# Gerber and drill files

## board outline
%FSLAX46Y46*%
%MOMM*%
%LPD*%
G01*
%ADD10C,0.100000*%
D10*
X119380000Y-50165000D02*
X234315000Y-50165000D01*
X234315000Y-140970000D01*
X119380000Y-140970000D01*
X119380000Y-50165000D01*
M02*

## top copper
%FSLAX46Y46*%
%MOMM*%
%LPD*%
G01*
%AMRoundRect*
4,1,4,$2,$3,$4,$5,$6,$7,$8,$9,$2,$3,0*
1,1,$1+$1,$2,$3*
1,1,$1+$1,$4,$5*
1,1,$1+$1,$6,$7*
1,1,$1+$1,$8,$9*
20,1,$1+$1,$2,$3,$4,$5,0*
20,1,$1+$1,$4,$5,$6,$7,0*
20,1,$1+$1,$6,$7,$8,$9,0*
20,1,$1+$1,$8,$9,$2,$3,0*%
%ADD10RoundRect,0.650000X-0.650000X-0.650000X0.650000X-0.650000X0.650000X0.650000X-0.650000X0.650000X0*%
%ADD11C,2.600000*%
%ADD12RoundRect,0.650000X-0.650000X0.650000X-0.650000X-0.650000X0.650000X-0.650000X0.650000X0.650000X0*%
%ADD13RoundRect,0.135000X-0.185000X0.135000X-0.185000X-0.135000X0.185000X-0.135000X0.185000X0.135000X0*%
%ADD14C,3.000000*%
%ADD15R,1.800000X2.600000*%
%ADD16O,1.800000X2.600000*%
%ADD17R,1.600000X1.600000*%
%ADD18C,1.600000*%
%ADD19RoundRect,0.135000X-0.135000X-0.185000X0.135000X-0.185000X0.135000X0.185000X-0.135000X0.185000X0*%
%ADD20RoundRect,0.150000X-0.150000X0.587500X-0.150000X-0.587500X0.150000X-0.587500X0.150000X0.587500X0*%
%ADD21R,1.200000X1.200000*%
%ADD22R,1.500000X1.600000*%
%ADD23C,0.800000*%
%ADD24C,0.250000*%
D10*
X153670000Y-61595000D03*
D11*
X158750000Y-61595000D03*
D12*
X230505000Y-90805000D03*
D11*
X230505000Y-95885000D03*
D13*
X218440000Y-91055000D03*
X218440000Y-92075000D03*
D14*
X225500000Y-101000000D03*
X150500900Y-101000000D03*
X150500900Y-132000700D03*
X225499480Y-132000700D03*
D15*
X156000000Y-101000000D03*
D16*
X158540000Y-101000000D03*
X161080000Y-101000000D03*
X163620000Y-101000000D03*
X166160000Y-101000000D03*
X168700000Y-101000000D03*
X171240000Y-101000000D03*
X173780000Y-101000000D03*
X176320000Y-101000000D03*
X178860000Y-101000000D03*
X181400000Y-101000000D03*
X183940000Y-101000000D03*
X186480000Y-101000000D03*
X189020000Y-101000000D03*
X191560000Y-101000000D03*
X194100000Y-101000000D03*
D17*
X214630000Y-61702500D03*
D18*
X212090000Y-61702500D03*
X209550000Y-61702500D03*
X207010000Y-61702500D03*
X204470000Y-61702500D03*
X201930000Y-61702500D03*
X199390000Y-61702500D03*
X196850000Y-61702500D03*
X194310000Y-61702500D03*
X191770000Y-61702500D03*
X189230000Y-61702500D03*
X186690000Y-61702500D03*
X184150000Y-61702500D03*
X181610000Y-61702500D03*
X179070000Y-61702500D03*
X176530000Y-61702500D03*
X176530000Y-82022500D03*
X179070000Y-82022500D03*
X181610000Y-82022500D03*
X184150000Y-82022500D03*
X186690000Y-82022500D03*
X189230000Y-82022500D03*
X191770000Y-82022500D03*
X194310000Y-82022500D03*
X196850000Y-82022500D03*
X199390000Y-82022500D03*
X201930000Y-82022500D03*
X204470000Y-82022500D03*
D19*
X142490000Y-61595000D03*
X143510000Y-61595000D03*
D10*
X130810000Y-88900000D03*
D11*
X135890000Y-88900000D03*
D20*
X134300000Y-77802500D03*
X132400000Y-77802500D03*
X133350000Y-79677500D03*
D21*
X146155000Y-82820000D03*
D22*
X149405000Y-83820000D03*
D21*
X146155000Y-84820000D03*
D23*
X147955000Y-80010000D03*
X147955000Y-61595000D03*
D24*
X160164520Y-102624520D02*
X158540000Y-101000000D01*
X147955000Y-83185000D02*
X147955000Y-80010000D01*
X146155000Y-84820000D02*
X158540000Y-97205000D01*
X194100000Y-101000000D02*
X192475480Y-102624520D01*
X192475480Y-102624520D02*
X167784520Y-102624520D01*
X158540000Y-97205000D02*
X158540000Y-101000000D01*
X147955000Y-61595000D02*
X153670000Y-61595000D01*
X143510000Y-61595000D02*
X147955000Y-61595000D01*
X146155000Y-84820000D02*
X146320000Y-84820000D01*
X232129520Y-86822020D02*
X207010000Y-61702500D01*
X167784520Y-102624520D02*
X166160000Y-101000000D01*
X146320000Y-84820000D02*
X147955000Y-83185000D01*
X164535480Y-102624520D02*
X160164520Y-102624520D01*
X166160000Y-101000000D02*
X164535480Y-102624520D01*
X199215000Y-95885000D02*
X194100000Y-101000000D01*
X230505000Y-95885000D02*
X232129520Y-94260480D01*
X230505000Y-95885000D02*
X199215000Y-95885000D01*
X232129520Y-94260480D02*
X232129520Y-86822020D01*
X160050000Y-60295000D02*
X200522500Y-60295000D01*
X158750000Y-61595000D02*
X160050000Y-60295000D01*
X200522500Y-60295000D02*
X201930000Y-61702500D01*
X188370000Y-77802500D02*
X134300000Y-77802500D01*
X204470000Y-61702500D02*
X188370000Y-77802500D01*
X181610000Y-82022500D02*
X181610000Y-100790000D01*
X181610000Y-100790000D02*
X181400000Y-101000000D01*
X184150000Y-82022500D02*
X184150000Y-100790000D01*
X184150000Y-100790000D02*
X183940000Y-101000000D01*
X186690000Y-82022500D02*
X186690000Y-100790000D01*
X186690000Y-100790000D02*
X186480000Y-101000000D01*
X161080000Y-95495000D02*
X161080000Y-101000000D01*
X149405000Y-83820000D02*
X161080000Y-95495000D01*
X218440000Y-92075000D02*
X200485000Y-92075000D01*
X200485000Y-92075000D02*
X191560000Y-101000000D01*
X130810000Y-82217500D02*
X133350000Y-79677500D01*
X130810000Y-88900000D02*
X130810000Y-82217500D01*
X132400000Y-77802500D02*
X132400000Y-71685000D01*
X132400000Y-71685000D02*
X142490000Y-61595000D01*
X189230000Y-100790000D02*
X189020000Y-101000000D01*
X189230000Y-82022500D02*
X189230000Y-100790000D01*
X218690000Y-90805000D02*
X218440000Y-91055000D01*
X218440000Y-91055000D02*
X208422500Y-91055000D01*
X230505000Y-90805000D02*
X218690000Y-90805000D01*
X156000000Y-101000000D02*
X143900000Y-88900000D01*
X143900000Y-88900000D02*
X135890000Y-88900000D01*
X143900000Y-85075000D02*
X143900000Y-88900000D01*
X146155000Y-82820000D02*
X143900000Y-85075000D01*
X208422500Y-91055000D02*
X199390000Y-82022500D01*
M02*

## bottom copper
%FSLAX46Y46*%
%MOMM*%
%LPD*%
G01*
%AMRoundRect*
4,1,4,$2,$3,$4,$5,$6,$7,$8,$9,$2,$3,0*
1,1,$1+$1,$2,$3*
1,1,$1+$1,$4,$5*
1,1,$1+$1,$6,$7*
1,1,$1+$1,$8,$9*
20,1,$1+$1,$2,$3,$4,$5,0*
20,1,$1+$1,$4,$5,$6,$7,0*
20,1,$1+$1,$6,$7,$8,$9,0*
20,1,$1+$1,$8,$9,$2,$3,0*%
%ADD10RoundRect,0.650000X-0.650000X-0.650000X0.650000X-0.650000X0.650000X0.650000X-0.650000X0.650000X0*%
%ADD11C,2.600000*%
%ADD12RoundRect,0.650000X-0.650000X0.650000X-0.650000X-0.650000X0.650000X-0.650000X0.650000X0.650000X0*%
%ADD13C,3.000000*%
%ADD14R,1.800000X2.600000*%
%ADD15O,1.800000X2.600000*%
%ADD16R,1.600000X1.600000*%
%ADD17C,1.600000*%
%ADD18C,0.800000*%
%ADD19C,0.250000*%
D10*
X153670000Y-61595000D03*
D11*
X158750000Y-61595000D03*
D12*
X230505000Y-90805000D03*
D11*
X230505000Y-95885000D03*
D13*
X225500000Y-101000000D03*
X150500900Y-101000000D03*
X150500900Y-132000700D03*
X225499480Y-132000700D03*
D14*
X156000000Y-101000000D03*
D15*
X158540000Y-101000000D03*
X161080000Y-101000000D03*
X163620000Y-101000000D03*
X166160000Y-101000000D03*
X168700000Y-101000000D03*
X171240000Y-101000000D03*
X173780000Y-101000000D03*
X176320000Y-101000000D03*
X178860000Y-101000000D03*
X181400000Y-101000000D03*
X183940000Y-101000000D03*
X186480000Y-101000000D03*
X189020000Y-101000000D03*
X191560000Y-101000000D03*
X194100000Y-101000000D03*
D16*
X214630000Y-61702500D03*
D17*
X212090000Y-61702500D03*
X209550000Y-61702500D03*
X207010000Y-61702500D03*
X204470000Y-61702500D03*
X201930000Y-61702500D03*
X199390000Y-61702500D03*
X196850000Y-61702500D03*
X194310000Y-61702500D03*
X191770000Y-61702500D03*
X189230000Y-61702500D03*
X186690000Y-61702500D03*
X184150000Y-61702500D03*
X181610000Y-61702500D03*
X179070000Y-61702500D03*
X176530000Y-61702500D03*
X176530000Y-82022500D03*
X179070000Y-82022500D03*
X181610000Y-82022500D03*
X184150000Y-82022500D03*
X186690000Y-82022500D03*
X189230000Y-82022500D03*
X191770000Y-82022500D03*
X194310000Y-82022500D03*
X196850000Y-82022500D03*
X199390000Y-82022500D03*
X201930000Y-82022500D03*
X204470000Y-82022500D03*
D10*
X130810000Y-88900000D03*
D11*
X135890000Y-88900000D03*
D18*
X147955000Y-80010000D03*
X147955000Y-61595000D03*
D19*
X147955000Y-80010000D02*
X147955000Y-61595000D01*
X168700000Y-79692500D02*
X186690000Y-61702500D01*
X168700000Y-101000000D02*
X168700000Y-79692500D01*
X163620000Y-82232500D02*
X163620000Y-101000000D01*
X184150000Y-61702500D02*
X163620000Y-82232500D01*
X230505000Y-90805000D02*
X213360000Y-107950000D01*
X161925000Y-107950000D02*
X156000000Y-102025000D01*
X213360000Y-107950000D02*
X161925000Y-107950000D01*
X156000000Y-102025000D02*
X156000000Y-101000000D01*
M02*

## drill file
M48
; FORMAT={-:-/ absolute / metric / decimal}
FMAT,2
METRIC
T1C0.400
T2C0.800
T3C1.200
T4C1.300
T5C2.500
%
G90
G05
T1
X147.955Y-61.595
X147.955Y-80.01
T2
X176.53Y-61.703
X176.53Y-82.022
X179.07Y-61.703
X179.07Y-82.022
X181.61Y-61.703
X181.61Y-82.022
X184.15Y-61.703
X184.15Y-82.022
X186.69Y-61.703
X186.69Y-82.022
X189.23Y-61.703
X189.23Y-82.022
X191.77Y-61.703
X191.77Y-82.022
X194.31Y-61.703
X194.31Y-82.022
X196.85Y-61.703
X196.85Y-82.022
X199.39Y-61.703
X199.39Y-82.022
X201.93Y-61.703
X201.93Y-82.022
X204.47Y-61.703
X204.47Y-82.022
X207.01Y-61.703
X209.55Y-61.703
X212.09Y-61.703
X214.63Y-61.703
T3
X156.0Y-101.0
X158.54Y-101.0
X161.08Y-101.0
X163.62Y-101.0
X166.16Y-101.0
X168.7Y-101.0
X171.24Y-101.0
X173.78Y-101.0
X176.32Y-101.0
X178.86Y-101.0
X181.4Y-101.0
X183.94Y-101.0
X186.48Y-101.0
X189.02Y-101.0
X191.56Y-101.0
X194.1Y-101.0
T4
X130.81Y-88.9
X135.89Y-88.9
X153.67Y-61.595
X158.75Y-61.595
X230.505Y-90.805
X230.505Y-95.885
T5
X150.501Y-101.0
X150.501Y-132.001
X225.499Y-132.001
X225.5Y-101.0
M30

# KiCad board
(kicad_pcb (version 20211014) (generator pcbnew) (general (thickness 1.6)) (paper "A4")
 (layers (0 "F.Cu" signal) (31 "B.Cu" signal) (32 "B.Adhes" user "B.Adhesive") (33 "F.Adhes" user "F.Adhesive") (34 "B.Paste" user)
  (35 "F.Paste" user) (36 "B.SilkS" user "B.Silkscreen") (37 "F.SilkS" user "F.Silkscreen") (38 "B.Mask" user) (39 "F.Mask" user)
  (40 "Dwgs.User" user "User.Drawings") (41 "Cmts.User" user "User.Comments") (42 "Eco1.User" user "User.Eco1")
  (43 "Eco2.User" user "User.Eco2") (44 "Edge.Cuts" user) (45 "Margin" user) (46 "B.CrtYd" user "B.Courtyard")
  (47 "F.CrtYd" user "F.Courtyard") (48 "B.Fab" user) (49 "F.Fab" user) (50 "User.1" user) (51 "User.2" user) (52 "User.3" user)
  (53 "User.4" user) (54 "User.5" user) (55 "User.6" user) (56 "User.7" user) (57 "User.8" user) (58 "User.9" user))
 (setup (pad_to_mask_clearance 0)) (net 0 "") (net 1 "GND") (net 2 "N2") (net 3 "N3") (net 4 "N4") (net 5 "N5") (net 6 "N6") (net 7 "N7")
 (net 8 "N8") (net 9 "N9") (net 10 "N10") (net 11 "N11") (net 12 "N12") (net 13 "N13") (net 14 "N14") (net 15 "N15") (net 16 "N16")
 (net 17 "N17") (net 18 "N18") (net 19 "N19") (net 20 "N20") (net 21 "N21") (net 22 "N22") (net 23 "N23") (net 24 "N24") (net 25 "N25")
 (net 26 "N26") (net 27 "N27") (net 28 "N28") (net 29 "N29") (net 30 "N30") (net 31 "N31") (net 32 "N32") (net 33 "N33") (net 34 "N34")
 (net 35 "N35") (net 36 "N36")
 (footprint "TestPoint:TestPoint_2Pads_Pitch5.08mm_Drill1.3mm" (layer "F.Cu") (at 153.67 61.595)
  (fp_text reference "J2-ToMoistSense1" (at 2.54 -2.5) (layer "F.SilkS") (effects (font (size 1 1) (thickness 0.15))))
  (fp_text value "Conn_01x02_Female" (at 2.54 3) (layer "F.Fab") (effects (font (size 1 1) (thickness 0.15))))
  (pad "1" thru_hole roundrect (at 0 0) (size 2.6 2.6) (drill 1.3) (layers *.Cu *.Mask) (roundrect_rratio 0.25) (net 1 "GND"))
  (pad "2" thru_hole circle (at 5.08 0) (size 2.6 2.6) (drill 1.3) (layers *.Cu *.Mask) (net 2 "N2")))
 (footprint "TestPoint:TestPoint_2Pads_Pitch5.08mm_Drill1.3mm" (layer "F.Cu") (at 230.505 90.805 -90)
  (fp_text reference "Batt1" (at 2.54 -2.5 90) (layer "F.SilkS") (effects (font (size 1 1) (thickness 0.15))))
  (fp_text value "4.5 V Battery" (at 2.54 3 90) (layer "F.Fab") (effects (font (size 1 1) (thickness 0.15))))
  (pad "1" thru_hole roundrect (at 0 0 270) (size 2.6 2.6) (drill 1.3) (layers *.Cu *.Mask) (roundrect_rratio 0.25) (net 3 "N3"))
  (pad "2" thru_hole circle (at 5.08 0 270) (size 2.6 2.6) (drill 1.3) (layers *.Cu *.Mask) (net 1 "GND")))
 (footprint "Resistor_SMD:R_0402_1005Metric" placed (layer "F.Cu") (at 218.44 91.565 -90)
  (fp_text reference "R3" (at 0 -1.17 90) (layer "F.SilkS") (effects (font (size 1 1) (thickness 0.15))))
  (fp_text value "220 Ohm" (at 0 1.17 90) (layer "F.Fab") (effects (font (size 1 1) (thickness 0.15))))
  (pad "1" smd roundrect (at -0.51 0 270) (size 0.54 0.64) (layers "F.Cu" "F.Paste" "F.Mask") (roundrect_rratio 0.25) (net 3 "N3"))
  (pad "2" smd roundrect (at 0.51 0 270) (size 0.54 0.64) (layers "F.Cu" "F.Paste" "F.Mask") (roundrect_rratio 0.25) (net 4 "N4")))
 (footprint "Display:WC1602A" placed (layer "F.Cu") (at 156 101)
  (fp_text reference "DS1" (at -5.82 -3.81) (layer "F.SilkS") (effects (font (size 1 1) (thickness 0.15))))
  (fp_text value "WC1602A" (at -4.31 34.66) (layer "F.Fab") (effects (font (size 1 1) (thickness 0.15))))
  (pad "" thru_hole circle (at 69.5 0) (size 3 3) (drill 2.5) (layers *.Cu *.Mask))
  (pad "" thru_hole circle (at -5.4991 0) (size 3 3) (drill 2.5) (layers *.Cu *.Mask))
  (pad "" thru_hole circle (at -5.4991 31.0007) (size 3 3) (drill 2.5) (layers *.Cu *.Mask))
  (pad "" thru_hole circle (at 69.49948 31.0007) (size 3 3) (drill 2.5) (layers *.Cu *.Mask))
  (pad "1" thru_hole rect (at 0 0) (size 1.8 2.6) (drill 1.2) (layers *.Cu *.Mask) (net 3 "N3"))
  (pad "2" thru_hole oval (at 2.54 0) (size 1.8 2.6) (drill 1.2) (layers *.Cu *.Mask) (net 1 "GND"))
  (pad "3" thru_hole oval (at 5.08 0) (size 1.8 2.6) (drill 1.2) (layers *.Cu *.Mask) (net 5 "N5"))
  (pad "4" thru_hole oval (at 7.62 0) (size 1.8 2.6) (drill 1.2) (layers *.Cu *.Mask) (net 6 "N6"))
  (pad "5" thru_hole oval (at 10.16 0) (size 1.8 2.6) (drill 1.2) (layers *.Cu *.Mask) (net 1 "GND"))
  (pad "6" thru_hole oval (at 12.7 0) (size 1.8 2.6) (drill 1.2) (layers *.Cu *.Mask) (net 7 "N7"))
  (pad "7" thru_hole oval (at 15.24 0) (size 1.8 2.6) (drill 1.2) (layers *.Cu *.Mask) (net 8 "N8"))
  (pad "8" thru_hole oval (at 17.78 0) (size 1.8 2.6) (drill 1.2) (layers *.Cu *.Mask) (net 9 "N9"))
  (pad "9" thru_hole oval (at 20.32 0) (size 1.8 2.6) (drill 1.2) (layers *.Cu *.Mask) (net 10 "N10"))
  (pad "10" thru_hole oval (at 22.86 0) (size 1.8 2.6) (drill 1.2) (layers *.Cu *.Mask) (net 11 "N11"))
  (pad "11" thru_hole oval (at 25.4 0) (size 1.8 2.6) (drill 1.2) (layers *.Cu *.Mask) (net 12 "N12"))
  (pad "12" thru_hole oval (at 27.94 0) (size 1.8 2.6) (drill 1.2) (layers *.Cu *.Mask) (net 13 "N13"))
  (pad "13" thru_hole oval (at 30.48 0) (size 1.8 2.6) (drill 1.2) (layers *.Cu *.Mask) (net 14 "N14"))
  (pad "14" thru_hole oval (at 33.02 0) (size 1.8 2.6) (drill 1.2) (layers *.Cu *.Mask) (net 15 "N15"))
  (pad "15" thru_hole oval (at 35.56 0) (size 1.8 2.6) (drill 1.2) (layers *.Cu *.Mask) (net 4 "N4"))
  (pad "16" thru_hole oval (at 38.1 0) (size 1.8 2.6) (drill 1.2) (layers *.Cu *.Mask) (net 1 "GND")))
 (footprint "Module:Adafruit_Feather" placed (layer "F.Cu") (at 214.63 61.7025 -90)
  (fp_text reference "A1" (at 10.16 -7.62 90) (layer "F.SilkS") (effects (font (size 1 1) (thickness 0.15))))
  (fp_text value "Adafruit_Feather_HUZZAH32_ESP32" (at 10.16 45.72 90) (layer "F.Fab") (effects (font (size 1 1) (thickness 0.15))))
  (pad "1" thru_hole rect (at 0 0 90) (size 1.6 1.6) (drill 0.8) (layers *.Cu *.Mask) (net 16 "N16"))
  (pad "2" thru_hole circle (at 0 2.54 90) (size 1.6 1.6) (drill 0.8) (layers *.Cu *.Mask) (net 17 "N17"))
  (pad "3" thru_hole circle (at 0 5.08 90) (size 1.6 1.6) (drill 0.8) (layers *.Cu *.Mask) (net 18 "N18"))
  (pad "4" thru_hole circle (at 0 7.62 90) (size 1.6 1.6) (drill 0.8) (layers *.Cu *.Mask) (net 1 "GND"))
  (pad "5" thru_hole circle (at 0 10.16 90) (size 1.6 1.6) (drill 0.8) (layers *.Cu *.Mask) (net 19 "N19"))
  (pad "6" thru_hole circle (at 0 12.7 90) (size 1.6 1.6) (drill 0.8) (layers *.Cu *.Mask) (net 2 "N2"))
  (pad "7" thru_hole circle (at 0 15.24 90) (size 1.6 1.6) (drill 0.8) (layers *.Cu *.Mask) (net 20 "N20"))
  (pad "8" thru_hole circle (at 0 17.78 90) (size 1.6 1.6) (drill 0.8) (layers *.Cu *.Mask) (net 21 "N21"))
  (pad "9" thru_hole circle (at 0 20.32 90) (size 1.6 1.6) (drill 0.8) (layers *.Cu *.Mask) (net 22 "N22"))
  (pad "10" thru_hole circle (at 0 22.86 90) (size 1.6 1.6) (drill 0.8) (layers *.Cu *.Mask) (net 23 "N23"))
  (pad "11" thru_hole circle (at 0 25.4 90) (size 1.6 1.6) (drill 0.8) (layers *.Cu *.Mask) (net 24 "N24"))
  (pad "12" thru_hole circle (at 0 27.94 90) (size 1.6 1.6) (drill 0.8) (layers *.Cu *.Mask) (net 7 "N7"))
  (pad "13" thru_hole circle (at 0 30.48 90) (size 1.6 1.6) (drill 0.8) (layers *.Cu *.Mask) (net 6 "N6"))
  (pad "14" thru_hole circle (at 0 33.02 90) (size 1.6 1.6) (drill 0.8) (layers *.Cu *.Mask) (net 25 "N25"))
  (pad "15" thru_hole circle (at 0 35.56 90) (size 1.6 1.6) (drill 0.8) (layers *.Cu *.Mask) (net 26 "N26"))
  (pad "16" thru_hole circle (at 0 38.1 90) (size 1.6 1.6) (drill 0.8) (layers *.Cu *.Mask) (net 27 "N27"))
  (pad "17" thru_hole circle (at 20.32 38.1 90) (size 1.6 1.6) (drill 0.8) (layers *.Cu *.Mask) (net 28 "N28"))
  (pad "18" thru_hole circle (at 20.32 35.56 90) (size 1.6 1.6) (drill 0.8) (layers *.Cu *.Mask) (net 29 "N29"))
  (pad "19" thru_hole circle (at 20.32 33.02 90) (size 1.6 1.6) (drill 0.8) (layers *.Cu *.Mask) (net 12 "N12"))
  (pad "20" thru_hole circle (at 20.32 30.48 90) (size 1.6 1.6) (drill 0.8) (layers *.Cu *.Mask) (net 13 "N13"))
  (pad "21" thru_hole circle (at 20.32 27.94 90) (size 1.6 1.6) (drill 0.8) (layers *.Cu *.Mask) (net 14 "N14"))
  (pad "22" thru_hole circle (at 20.32 25.4 90) (size 1.6 1.6) (drill 0.8) (layers *.Cu *.Mask) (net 15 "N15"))
  (pad "23" thru_hole circle (at 20.32 22.86 90) (size 1.6 1.6) (drill 0.8) (layers *.Cu *.Mask) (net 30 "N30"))
  (pad "24" thru_hole circle (at 20.32 20.32 90) (size 1.6 1.6) (drill 0.8) (layers *.Cu *.Mask) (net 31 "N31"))
  (pad "25" thru_hole circle (at 20.32 17.78 90) (size 1.6 1.6) (drill 0.8) (layers *.Cu *.Mask) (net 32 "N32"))
  (pad "26" thru_hole circle (at 20.32 15.24 90) (size 1.6 1.6) (drill 0.8) (layers *.Cu *.Mask) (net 3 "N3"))
  (pad "27" thru_hole circle (at 20.32 12.7 90) (size 1.6 1.6) (drill 0.8) (layers *.Cu *.Mask) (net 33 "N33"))
  (pad "28" thru_hole circle (at 20.32 10.16 90) (size 1.6 1.6) (drill 0.8) (layers *.Cu *.Mask) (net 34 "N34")))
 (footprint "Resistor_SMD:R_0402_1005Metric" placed (layer "F.Cu") (at 143 61.595)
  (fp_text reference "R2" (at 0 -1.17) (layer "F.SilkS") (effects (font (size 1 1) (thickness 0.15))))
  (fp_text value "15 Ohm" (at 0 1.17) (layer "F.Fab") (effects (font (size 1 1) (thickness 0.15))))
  (pad "1" smd roundrect (at -0.51 0) (size 0.54 0.64) (layers "F.Cu" "F.Paste" "F.Mask") (roundrect_rratio 0.25) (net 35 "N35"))
  (pad "2" smd roundrect (at 0.51 0) (size 0.54 0.64) (layers "F.Cu" "F.Paste" "F.Mask") (roundrect_rratio 0.25) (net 1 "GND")))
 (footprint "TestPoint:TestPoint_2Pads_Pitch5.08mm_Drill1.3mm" (layer "F.Cu") (at 130.81 88.9)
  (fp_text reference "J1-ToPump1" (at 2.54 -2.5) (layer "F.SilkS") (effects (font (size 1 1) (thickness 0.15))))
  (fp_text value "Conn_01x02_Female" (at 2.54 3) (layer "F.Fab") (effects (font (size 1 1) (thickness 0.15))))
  (pad "1" thru_hole roundrect (at 0 0) (size 2.6 2.6) (drill 1.3) (layers *.Cu *.Mask) (roundrect_rratio 0.25) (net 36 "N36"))
  (pad "2" thru_hole circle (at 5.08 0) (size 2.6 2.6) (drill 1.3) (layers *.Cu *.Mask) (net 3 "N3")))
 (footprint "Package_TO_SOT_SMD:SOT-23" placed (layer "F.Cu") (at 133.35 78.74 -90)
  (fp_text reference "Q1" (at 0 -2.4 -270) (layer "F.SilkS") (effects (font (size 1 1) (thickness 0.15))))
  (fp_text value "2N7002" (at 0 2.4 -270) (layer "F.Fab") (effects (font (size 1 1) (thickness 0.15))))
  (pad "1" smd roundrect (at -0.9375 -0.95 270) (size 1.475 0.6) (layers "F.Cu" "F.Paste" "F.Mask") (roundrect_rratio 0.25) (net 19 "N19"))
  (pad "2" smd roundrect (at -0.9375 0.95 270) (size 1.475 0.6) (layers "F.Cu" "F.Paste" "F.Mask") (roundrect_rratio 0.25) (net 35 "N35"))
  (pad "3" smd roundrect (at 0.9375 0 270) (size 1.475 0.6) (layers "F.Cu" "F.Paste" "F.Mask") (roundrect_rratio 0.25) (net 36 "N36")))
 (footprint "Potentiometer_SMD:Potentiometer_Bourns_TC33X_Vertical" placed (layer "F.Cu") (at 147.955 83.82)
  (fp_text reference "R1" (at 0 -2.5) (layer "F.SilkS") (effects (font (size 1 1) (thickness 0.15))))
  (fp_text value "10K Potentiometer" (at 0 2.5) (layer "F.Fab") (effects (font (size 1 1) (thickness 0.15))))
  (pad "1" smd rect (at -1.8 -1) (size 1.2 1.2) (layers "F.Cu" "F.Paste" "F.Mask") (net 3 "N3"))
  (pad "2" smd rect (at 1.45 0) (size 1.5 1.6) (layers "F.Cu" "F.Paste" "F.Mask") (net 5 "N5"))
  (pad "3" smd rect (at -1.8 1) (size 1.2 1.2) (layers "F.Cu" "F.Paste" "F.Mask") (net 1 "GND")))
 (gr_rect (start 119.38 140.97) (end 234.315 50.165) (layer "Edge.Cuts") (width 0.1) (fill none))
 (segment (start 160.16452 102.62452) (end 158.54 101) (width 0.25) (layer "F.Cu") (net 1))
 (segment (start 147.955 83.185) (end 147.955 80.01) (width 0.25) (layer "F.Cu") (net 1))
 (segment (start 146.155 84.82) (end 158.54 97.205) (width 0.25) (layer "F.Cu") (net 1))
 (segment (start 194.1 101) (end 192.47548 102.62452) (width 0.25) (layer "F.Cu") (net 1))
 (segment (start 192.47548 102.62452) (end 167.78452 102.62452) (width 0.25) (layer "F.Cu") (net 1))
 (segment (start 158.54 97.205) (end 158.54 101) (width 0.25) (layer "F.Cu") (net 1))
 (segment (start 147.955 61.595) (end 153.67 61.595) (width 0.25) (layer "F.Cu") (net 1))
 (segment (start 143.51 61.595) (end 147.955 61.595) (width 0.25) (layer "F.Cu") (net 1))
 (segment (start 146.155 84.82) (end 146.32 84.82) (width 0.25) (layer "F.Cu") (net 1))
 (segment (start 232.12952 86.82202) (end 207.01 61.7025) (width 0.25) (layer "F.Cu") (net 1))
 (segment (start 167.78452 102.62452) (end 166.16 101) (width 0.25) (layer "F.Cu") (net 1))
 (segment (start 146.32 84.82) (end 147.955 83.185) (width 0.25) (layer "F.Cu") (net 1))
 (segment (start 164.53548 102.62452) (end 160.16452 102.62452) (width 0.25) (layer "F.Cu") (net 1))
 (segment (start 166.16 101) (end 164.53548 102.62452) (width 0.25) (layer "F.Cu") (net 1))
 (segment (start 199.215 95.885) (end 194.1 101) (width 0.25) (layer "F.Cu") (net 1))
 (segment (start 230.505 95.885) (end 232.12952 94.26048) (width 0.25) (layer "F.Cu") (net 1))
 (segment (start 230.505 95.885) (end 199.215 95.885) (width 0.25) (layer "F.Cu") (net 1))
 (segment (start 232.12952 94.26048) (end 232.12952 86.82202) (width 0.25) (layer "F.Cu") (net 1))
 (via (at 147.955 80.01) (size 0.8) (drill 0.4) (layers "F.Cu" "B.Cu") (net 1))
 (via (at 147.955 61.595) (size 0.8) (drill 0.4) (layers "F.Cu" "B.Cu") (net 1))
 (segment (start 147.955 80.01) (end 147.955 61.595) (width 0.25) (layer "B.Cu") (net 1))
 (segment (start 160.05 60.295) (end 200.5225 60.295) (width 0.25) (layer "F.Cu") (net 2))
 (segment (start 158.75 61.595) (end 160.05 60.295) (width 0.25) (layer "F.Cu") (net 2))
 (segment (start 200.5225 60.295) (end 201.93 61.7025) (width 0.25) (layer "F.Cu") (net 2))
 (segment (start 188.37 77.8025) (end 134.3 77.8025) (width 0.25) (layer "F.Cu") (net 19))
 (segment (start 204.47 61.7025) (end 188.37 77.8025) (width 0.25) (layer "F.Cu") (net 19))
 (segment (start 181.61 82.0225) (end 181.61 100.79) (width 0.25) (layer "F.Cu") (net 12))
 (segment (start 181.61 100.79) (end 181.4 101) (width 0.25) (layer "F.Cu") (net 12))
 (segment (start 184.15 82.0225) (end 184.15 100.79) (width 0.25) (layer "F.Cu") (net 13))
 (segment (start 184.15 100.79) (end 183.94 101) (width 0.25) (layer "F.Cu") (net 13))
 (segment (start 186.69 82.0225) (end 186.69 100.79) (width 0.25) (layer "F.Cu") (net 14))
 (segment (start 186.69 100.79) (end 186.48 101) (width 0.25) (layer "F.Cu") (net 14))
 (segment (start 161.08 95.495) (end 161.08 101) (width 0.25) (layer "F.Cu") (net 5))
 (segment (start 149.405 83.82) (end 161.08 95.495) (width 0.25) (layer "F.Cu") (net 5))
 (segment (start 218.44 92.075) (end 200.485 92.075) (width 0.25) (layer "F.Cu") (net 4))
 (segment (start 200.485 92.075) (end 191.56 101) (width 0.25) (layer "F.Cu") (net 4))
 (segment (start 130.81 82.2175) (end 133.35 79.6775) (width 0.25) (layer "F.Cu") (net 36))
 (segment (start 130.81 88.9) (end 130.81 82.2175) (width 0.25) (layer "F.Cu") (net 36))
 (segment (start 132.4 77.8025) (end 132.4 71.685) (width 0.25) (layer "F.Cu") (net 35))
 (segment (start 132.4 71.685) (end 142.49 61.595) (width 0.25) (layer "F.Cu") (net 35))
 (segment (start 168.7 79.6925) (end 186.69 61.7025) (width 0.25) (layer "B.Cu") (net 7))
 (segment (start 168.7 101) (end 168.7 79.6925) (width 0.25) (layer "B.Cu") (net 7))
 (segment (start 163.62 82.2325) (end 163.62 101) (width 0.25) (layer "B.Cu") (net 6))
 (segment (start 184.15 61.7025) (end 163.62 82.2325) (width 0.25) (layer "B.Cu") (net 6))
 (segment (start 189.23 100.79) (end 189.02 101) (width 0.25) (layer "F.Cu") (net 15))
 (segment (start 189.23 82.0225) (end 189.23 100.79) (width 0.25) (layer "F.Cu") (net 15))
 (segment (start 218.69 90.805) (end 218.44 91.055) (width 0.25) (layer "F.Cu") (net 3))
 (segment (start 218.44 91.055) (end 208.4225 91.055) (width 0.25) (layer "F.Cu") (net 3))
 (segment (start 230.505 90.805) (end 218.69 90.805) (width 0.25) (layer "F.Cu") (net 3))
 (segment (start 156 101) (end 143.9 88.9) (width 0.25) (layer "F.Cu") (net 3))
 (segment (start 143.9 88.9) (end 135.89 88.9) (width 0.25) (layer "F.Cu") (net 3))
 (segment (start 143.9 85.075) (end 143.9 88.9) (width 0.25) (layer "F.Cu") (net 3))
 (segment (start 146.155 82.82) (end 143.9 85.075) (width 0.25) (layer "F.Cu") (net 3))
 (segment (start 208.4225 91.055) (end 199.39 82.0225) (width 0.25) (layer "F.Cu") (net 3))
 (segment (start 230.505 90.805) (end 213.36 107.95) (width 0.25) (layer "B.Cu") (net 3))
 (segment (start 161.925 107.95) (end 156 102.025) (width 0.25) (layer "B.Cu") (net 3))
 (segment (start 213.36 107.95) (end 161.925 107.95) (width 0.25) (layer "B.Cu") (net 3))
 (segment (start 156 102.025) (end 156 101) (width 0.25) (layer "B.Cu") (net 3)))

